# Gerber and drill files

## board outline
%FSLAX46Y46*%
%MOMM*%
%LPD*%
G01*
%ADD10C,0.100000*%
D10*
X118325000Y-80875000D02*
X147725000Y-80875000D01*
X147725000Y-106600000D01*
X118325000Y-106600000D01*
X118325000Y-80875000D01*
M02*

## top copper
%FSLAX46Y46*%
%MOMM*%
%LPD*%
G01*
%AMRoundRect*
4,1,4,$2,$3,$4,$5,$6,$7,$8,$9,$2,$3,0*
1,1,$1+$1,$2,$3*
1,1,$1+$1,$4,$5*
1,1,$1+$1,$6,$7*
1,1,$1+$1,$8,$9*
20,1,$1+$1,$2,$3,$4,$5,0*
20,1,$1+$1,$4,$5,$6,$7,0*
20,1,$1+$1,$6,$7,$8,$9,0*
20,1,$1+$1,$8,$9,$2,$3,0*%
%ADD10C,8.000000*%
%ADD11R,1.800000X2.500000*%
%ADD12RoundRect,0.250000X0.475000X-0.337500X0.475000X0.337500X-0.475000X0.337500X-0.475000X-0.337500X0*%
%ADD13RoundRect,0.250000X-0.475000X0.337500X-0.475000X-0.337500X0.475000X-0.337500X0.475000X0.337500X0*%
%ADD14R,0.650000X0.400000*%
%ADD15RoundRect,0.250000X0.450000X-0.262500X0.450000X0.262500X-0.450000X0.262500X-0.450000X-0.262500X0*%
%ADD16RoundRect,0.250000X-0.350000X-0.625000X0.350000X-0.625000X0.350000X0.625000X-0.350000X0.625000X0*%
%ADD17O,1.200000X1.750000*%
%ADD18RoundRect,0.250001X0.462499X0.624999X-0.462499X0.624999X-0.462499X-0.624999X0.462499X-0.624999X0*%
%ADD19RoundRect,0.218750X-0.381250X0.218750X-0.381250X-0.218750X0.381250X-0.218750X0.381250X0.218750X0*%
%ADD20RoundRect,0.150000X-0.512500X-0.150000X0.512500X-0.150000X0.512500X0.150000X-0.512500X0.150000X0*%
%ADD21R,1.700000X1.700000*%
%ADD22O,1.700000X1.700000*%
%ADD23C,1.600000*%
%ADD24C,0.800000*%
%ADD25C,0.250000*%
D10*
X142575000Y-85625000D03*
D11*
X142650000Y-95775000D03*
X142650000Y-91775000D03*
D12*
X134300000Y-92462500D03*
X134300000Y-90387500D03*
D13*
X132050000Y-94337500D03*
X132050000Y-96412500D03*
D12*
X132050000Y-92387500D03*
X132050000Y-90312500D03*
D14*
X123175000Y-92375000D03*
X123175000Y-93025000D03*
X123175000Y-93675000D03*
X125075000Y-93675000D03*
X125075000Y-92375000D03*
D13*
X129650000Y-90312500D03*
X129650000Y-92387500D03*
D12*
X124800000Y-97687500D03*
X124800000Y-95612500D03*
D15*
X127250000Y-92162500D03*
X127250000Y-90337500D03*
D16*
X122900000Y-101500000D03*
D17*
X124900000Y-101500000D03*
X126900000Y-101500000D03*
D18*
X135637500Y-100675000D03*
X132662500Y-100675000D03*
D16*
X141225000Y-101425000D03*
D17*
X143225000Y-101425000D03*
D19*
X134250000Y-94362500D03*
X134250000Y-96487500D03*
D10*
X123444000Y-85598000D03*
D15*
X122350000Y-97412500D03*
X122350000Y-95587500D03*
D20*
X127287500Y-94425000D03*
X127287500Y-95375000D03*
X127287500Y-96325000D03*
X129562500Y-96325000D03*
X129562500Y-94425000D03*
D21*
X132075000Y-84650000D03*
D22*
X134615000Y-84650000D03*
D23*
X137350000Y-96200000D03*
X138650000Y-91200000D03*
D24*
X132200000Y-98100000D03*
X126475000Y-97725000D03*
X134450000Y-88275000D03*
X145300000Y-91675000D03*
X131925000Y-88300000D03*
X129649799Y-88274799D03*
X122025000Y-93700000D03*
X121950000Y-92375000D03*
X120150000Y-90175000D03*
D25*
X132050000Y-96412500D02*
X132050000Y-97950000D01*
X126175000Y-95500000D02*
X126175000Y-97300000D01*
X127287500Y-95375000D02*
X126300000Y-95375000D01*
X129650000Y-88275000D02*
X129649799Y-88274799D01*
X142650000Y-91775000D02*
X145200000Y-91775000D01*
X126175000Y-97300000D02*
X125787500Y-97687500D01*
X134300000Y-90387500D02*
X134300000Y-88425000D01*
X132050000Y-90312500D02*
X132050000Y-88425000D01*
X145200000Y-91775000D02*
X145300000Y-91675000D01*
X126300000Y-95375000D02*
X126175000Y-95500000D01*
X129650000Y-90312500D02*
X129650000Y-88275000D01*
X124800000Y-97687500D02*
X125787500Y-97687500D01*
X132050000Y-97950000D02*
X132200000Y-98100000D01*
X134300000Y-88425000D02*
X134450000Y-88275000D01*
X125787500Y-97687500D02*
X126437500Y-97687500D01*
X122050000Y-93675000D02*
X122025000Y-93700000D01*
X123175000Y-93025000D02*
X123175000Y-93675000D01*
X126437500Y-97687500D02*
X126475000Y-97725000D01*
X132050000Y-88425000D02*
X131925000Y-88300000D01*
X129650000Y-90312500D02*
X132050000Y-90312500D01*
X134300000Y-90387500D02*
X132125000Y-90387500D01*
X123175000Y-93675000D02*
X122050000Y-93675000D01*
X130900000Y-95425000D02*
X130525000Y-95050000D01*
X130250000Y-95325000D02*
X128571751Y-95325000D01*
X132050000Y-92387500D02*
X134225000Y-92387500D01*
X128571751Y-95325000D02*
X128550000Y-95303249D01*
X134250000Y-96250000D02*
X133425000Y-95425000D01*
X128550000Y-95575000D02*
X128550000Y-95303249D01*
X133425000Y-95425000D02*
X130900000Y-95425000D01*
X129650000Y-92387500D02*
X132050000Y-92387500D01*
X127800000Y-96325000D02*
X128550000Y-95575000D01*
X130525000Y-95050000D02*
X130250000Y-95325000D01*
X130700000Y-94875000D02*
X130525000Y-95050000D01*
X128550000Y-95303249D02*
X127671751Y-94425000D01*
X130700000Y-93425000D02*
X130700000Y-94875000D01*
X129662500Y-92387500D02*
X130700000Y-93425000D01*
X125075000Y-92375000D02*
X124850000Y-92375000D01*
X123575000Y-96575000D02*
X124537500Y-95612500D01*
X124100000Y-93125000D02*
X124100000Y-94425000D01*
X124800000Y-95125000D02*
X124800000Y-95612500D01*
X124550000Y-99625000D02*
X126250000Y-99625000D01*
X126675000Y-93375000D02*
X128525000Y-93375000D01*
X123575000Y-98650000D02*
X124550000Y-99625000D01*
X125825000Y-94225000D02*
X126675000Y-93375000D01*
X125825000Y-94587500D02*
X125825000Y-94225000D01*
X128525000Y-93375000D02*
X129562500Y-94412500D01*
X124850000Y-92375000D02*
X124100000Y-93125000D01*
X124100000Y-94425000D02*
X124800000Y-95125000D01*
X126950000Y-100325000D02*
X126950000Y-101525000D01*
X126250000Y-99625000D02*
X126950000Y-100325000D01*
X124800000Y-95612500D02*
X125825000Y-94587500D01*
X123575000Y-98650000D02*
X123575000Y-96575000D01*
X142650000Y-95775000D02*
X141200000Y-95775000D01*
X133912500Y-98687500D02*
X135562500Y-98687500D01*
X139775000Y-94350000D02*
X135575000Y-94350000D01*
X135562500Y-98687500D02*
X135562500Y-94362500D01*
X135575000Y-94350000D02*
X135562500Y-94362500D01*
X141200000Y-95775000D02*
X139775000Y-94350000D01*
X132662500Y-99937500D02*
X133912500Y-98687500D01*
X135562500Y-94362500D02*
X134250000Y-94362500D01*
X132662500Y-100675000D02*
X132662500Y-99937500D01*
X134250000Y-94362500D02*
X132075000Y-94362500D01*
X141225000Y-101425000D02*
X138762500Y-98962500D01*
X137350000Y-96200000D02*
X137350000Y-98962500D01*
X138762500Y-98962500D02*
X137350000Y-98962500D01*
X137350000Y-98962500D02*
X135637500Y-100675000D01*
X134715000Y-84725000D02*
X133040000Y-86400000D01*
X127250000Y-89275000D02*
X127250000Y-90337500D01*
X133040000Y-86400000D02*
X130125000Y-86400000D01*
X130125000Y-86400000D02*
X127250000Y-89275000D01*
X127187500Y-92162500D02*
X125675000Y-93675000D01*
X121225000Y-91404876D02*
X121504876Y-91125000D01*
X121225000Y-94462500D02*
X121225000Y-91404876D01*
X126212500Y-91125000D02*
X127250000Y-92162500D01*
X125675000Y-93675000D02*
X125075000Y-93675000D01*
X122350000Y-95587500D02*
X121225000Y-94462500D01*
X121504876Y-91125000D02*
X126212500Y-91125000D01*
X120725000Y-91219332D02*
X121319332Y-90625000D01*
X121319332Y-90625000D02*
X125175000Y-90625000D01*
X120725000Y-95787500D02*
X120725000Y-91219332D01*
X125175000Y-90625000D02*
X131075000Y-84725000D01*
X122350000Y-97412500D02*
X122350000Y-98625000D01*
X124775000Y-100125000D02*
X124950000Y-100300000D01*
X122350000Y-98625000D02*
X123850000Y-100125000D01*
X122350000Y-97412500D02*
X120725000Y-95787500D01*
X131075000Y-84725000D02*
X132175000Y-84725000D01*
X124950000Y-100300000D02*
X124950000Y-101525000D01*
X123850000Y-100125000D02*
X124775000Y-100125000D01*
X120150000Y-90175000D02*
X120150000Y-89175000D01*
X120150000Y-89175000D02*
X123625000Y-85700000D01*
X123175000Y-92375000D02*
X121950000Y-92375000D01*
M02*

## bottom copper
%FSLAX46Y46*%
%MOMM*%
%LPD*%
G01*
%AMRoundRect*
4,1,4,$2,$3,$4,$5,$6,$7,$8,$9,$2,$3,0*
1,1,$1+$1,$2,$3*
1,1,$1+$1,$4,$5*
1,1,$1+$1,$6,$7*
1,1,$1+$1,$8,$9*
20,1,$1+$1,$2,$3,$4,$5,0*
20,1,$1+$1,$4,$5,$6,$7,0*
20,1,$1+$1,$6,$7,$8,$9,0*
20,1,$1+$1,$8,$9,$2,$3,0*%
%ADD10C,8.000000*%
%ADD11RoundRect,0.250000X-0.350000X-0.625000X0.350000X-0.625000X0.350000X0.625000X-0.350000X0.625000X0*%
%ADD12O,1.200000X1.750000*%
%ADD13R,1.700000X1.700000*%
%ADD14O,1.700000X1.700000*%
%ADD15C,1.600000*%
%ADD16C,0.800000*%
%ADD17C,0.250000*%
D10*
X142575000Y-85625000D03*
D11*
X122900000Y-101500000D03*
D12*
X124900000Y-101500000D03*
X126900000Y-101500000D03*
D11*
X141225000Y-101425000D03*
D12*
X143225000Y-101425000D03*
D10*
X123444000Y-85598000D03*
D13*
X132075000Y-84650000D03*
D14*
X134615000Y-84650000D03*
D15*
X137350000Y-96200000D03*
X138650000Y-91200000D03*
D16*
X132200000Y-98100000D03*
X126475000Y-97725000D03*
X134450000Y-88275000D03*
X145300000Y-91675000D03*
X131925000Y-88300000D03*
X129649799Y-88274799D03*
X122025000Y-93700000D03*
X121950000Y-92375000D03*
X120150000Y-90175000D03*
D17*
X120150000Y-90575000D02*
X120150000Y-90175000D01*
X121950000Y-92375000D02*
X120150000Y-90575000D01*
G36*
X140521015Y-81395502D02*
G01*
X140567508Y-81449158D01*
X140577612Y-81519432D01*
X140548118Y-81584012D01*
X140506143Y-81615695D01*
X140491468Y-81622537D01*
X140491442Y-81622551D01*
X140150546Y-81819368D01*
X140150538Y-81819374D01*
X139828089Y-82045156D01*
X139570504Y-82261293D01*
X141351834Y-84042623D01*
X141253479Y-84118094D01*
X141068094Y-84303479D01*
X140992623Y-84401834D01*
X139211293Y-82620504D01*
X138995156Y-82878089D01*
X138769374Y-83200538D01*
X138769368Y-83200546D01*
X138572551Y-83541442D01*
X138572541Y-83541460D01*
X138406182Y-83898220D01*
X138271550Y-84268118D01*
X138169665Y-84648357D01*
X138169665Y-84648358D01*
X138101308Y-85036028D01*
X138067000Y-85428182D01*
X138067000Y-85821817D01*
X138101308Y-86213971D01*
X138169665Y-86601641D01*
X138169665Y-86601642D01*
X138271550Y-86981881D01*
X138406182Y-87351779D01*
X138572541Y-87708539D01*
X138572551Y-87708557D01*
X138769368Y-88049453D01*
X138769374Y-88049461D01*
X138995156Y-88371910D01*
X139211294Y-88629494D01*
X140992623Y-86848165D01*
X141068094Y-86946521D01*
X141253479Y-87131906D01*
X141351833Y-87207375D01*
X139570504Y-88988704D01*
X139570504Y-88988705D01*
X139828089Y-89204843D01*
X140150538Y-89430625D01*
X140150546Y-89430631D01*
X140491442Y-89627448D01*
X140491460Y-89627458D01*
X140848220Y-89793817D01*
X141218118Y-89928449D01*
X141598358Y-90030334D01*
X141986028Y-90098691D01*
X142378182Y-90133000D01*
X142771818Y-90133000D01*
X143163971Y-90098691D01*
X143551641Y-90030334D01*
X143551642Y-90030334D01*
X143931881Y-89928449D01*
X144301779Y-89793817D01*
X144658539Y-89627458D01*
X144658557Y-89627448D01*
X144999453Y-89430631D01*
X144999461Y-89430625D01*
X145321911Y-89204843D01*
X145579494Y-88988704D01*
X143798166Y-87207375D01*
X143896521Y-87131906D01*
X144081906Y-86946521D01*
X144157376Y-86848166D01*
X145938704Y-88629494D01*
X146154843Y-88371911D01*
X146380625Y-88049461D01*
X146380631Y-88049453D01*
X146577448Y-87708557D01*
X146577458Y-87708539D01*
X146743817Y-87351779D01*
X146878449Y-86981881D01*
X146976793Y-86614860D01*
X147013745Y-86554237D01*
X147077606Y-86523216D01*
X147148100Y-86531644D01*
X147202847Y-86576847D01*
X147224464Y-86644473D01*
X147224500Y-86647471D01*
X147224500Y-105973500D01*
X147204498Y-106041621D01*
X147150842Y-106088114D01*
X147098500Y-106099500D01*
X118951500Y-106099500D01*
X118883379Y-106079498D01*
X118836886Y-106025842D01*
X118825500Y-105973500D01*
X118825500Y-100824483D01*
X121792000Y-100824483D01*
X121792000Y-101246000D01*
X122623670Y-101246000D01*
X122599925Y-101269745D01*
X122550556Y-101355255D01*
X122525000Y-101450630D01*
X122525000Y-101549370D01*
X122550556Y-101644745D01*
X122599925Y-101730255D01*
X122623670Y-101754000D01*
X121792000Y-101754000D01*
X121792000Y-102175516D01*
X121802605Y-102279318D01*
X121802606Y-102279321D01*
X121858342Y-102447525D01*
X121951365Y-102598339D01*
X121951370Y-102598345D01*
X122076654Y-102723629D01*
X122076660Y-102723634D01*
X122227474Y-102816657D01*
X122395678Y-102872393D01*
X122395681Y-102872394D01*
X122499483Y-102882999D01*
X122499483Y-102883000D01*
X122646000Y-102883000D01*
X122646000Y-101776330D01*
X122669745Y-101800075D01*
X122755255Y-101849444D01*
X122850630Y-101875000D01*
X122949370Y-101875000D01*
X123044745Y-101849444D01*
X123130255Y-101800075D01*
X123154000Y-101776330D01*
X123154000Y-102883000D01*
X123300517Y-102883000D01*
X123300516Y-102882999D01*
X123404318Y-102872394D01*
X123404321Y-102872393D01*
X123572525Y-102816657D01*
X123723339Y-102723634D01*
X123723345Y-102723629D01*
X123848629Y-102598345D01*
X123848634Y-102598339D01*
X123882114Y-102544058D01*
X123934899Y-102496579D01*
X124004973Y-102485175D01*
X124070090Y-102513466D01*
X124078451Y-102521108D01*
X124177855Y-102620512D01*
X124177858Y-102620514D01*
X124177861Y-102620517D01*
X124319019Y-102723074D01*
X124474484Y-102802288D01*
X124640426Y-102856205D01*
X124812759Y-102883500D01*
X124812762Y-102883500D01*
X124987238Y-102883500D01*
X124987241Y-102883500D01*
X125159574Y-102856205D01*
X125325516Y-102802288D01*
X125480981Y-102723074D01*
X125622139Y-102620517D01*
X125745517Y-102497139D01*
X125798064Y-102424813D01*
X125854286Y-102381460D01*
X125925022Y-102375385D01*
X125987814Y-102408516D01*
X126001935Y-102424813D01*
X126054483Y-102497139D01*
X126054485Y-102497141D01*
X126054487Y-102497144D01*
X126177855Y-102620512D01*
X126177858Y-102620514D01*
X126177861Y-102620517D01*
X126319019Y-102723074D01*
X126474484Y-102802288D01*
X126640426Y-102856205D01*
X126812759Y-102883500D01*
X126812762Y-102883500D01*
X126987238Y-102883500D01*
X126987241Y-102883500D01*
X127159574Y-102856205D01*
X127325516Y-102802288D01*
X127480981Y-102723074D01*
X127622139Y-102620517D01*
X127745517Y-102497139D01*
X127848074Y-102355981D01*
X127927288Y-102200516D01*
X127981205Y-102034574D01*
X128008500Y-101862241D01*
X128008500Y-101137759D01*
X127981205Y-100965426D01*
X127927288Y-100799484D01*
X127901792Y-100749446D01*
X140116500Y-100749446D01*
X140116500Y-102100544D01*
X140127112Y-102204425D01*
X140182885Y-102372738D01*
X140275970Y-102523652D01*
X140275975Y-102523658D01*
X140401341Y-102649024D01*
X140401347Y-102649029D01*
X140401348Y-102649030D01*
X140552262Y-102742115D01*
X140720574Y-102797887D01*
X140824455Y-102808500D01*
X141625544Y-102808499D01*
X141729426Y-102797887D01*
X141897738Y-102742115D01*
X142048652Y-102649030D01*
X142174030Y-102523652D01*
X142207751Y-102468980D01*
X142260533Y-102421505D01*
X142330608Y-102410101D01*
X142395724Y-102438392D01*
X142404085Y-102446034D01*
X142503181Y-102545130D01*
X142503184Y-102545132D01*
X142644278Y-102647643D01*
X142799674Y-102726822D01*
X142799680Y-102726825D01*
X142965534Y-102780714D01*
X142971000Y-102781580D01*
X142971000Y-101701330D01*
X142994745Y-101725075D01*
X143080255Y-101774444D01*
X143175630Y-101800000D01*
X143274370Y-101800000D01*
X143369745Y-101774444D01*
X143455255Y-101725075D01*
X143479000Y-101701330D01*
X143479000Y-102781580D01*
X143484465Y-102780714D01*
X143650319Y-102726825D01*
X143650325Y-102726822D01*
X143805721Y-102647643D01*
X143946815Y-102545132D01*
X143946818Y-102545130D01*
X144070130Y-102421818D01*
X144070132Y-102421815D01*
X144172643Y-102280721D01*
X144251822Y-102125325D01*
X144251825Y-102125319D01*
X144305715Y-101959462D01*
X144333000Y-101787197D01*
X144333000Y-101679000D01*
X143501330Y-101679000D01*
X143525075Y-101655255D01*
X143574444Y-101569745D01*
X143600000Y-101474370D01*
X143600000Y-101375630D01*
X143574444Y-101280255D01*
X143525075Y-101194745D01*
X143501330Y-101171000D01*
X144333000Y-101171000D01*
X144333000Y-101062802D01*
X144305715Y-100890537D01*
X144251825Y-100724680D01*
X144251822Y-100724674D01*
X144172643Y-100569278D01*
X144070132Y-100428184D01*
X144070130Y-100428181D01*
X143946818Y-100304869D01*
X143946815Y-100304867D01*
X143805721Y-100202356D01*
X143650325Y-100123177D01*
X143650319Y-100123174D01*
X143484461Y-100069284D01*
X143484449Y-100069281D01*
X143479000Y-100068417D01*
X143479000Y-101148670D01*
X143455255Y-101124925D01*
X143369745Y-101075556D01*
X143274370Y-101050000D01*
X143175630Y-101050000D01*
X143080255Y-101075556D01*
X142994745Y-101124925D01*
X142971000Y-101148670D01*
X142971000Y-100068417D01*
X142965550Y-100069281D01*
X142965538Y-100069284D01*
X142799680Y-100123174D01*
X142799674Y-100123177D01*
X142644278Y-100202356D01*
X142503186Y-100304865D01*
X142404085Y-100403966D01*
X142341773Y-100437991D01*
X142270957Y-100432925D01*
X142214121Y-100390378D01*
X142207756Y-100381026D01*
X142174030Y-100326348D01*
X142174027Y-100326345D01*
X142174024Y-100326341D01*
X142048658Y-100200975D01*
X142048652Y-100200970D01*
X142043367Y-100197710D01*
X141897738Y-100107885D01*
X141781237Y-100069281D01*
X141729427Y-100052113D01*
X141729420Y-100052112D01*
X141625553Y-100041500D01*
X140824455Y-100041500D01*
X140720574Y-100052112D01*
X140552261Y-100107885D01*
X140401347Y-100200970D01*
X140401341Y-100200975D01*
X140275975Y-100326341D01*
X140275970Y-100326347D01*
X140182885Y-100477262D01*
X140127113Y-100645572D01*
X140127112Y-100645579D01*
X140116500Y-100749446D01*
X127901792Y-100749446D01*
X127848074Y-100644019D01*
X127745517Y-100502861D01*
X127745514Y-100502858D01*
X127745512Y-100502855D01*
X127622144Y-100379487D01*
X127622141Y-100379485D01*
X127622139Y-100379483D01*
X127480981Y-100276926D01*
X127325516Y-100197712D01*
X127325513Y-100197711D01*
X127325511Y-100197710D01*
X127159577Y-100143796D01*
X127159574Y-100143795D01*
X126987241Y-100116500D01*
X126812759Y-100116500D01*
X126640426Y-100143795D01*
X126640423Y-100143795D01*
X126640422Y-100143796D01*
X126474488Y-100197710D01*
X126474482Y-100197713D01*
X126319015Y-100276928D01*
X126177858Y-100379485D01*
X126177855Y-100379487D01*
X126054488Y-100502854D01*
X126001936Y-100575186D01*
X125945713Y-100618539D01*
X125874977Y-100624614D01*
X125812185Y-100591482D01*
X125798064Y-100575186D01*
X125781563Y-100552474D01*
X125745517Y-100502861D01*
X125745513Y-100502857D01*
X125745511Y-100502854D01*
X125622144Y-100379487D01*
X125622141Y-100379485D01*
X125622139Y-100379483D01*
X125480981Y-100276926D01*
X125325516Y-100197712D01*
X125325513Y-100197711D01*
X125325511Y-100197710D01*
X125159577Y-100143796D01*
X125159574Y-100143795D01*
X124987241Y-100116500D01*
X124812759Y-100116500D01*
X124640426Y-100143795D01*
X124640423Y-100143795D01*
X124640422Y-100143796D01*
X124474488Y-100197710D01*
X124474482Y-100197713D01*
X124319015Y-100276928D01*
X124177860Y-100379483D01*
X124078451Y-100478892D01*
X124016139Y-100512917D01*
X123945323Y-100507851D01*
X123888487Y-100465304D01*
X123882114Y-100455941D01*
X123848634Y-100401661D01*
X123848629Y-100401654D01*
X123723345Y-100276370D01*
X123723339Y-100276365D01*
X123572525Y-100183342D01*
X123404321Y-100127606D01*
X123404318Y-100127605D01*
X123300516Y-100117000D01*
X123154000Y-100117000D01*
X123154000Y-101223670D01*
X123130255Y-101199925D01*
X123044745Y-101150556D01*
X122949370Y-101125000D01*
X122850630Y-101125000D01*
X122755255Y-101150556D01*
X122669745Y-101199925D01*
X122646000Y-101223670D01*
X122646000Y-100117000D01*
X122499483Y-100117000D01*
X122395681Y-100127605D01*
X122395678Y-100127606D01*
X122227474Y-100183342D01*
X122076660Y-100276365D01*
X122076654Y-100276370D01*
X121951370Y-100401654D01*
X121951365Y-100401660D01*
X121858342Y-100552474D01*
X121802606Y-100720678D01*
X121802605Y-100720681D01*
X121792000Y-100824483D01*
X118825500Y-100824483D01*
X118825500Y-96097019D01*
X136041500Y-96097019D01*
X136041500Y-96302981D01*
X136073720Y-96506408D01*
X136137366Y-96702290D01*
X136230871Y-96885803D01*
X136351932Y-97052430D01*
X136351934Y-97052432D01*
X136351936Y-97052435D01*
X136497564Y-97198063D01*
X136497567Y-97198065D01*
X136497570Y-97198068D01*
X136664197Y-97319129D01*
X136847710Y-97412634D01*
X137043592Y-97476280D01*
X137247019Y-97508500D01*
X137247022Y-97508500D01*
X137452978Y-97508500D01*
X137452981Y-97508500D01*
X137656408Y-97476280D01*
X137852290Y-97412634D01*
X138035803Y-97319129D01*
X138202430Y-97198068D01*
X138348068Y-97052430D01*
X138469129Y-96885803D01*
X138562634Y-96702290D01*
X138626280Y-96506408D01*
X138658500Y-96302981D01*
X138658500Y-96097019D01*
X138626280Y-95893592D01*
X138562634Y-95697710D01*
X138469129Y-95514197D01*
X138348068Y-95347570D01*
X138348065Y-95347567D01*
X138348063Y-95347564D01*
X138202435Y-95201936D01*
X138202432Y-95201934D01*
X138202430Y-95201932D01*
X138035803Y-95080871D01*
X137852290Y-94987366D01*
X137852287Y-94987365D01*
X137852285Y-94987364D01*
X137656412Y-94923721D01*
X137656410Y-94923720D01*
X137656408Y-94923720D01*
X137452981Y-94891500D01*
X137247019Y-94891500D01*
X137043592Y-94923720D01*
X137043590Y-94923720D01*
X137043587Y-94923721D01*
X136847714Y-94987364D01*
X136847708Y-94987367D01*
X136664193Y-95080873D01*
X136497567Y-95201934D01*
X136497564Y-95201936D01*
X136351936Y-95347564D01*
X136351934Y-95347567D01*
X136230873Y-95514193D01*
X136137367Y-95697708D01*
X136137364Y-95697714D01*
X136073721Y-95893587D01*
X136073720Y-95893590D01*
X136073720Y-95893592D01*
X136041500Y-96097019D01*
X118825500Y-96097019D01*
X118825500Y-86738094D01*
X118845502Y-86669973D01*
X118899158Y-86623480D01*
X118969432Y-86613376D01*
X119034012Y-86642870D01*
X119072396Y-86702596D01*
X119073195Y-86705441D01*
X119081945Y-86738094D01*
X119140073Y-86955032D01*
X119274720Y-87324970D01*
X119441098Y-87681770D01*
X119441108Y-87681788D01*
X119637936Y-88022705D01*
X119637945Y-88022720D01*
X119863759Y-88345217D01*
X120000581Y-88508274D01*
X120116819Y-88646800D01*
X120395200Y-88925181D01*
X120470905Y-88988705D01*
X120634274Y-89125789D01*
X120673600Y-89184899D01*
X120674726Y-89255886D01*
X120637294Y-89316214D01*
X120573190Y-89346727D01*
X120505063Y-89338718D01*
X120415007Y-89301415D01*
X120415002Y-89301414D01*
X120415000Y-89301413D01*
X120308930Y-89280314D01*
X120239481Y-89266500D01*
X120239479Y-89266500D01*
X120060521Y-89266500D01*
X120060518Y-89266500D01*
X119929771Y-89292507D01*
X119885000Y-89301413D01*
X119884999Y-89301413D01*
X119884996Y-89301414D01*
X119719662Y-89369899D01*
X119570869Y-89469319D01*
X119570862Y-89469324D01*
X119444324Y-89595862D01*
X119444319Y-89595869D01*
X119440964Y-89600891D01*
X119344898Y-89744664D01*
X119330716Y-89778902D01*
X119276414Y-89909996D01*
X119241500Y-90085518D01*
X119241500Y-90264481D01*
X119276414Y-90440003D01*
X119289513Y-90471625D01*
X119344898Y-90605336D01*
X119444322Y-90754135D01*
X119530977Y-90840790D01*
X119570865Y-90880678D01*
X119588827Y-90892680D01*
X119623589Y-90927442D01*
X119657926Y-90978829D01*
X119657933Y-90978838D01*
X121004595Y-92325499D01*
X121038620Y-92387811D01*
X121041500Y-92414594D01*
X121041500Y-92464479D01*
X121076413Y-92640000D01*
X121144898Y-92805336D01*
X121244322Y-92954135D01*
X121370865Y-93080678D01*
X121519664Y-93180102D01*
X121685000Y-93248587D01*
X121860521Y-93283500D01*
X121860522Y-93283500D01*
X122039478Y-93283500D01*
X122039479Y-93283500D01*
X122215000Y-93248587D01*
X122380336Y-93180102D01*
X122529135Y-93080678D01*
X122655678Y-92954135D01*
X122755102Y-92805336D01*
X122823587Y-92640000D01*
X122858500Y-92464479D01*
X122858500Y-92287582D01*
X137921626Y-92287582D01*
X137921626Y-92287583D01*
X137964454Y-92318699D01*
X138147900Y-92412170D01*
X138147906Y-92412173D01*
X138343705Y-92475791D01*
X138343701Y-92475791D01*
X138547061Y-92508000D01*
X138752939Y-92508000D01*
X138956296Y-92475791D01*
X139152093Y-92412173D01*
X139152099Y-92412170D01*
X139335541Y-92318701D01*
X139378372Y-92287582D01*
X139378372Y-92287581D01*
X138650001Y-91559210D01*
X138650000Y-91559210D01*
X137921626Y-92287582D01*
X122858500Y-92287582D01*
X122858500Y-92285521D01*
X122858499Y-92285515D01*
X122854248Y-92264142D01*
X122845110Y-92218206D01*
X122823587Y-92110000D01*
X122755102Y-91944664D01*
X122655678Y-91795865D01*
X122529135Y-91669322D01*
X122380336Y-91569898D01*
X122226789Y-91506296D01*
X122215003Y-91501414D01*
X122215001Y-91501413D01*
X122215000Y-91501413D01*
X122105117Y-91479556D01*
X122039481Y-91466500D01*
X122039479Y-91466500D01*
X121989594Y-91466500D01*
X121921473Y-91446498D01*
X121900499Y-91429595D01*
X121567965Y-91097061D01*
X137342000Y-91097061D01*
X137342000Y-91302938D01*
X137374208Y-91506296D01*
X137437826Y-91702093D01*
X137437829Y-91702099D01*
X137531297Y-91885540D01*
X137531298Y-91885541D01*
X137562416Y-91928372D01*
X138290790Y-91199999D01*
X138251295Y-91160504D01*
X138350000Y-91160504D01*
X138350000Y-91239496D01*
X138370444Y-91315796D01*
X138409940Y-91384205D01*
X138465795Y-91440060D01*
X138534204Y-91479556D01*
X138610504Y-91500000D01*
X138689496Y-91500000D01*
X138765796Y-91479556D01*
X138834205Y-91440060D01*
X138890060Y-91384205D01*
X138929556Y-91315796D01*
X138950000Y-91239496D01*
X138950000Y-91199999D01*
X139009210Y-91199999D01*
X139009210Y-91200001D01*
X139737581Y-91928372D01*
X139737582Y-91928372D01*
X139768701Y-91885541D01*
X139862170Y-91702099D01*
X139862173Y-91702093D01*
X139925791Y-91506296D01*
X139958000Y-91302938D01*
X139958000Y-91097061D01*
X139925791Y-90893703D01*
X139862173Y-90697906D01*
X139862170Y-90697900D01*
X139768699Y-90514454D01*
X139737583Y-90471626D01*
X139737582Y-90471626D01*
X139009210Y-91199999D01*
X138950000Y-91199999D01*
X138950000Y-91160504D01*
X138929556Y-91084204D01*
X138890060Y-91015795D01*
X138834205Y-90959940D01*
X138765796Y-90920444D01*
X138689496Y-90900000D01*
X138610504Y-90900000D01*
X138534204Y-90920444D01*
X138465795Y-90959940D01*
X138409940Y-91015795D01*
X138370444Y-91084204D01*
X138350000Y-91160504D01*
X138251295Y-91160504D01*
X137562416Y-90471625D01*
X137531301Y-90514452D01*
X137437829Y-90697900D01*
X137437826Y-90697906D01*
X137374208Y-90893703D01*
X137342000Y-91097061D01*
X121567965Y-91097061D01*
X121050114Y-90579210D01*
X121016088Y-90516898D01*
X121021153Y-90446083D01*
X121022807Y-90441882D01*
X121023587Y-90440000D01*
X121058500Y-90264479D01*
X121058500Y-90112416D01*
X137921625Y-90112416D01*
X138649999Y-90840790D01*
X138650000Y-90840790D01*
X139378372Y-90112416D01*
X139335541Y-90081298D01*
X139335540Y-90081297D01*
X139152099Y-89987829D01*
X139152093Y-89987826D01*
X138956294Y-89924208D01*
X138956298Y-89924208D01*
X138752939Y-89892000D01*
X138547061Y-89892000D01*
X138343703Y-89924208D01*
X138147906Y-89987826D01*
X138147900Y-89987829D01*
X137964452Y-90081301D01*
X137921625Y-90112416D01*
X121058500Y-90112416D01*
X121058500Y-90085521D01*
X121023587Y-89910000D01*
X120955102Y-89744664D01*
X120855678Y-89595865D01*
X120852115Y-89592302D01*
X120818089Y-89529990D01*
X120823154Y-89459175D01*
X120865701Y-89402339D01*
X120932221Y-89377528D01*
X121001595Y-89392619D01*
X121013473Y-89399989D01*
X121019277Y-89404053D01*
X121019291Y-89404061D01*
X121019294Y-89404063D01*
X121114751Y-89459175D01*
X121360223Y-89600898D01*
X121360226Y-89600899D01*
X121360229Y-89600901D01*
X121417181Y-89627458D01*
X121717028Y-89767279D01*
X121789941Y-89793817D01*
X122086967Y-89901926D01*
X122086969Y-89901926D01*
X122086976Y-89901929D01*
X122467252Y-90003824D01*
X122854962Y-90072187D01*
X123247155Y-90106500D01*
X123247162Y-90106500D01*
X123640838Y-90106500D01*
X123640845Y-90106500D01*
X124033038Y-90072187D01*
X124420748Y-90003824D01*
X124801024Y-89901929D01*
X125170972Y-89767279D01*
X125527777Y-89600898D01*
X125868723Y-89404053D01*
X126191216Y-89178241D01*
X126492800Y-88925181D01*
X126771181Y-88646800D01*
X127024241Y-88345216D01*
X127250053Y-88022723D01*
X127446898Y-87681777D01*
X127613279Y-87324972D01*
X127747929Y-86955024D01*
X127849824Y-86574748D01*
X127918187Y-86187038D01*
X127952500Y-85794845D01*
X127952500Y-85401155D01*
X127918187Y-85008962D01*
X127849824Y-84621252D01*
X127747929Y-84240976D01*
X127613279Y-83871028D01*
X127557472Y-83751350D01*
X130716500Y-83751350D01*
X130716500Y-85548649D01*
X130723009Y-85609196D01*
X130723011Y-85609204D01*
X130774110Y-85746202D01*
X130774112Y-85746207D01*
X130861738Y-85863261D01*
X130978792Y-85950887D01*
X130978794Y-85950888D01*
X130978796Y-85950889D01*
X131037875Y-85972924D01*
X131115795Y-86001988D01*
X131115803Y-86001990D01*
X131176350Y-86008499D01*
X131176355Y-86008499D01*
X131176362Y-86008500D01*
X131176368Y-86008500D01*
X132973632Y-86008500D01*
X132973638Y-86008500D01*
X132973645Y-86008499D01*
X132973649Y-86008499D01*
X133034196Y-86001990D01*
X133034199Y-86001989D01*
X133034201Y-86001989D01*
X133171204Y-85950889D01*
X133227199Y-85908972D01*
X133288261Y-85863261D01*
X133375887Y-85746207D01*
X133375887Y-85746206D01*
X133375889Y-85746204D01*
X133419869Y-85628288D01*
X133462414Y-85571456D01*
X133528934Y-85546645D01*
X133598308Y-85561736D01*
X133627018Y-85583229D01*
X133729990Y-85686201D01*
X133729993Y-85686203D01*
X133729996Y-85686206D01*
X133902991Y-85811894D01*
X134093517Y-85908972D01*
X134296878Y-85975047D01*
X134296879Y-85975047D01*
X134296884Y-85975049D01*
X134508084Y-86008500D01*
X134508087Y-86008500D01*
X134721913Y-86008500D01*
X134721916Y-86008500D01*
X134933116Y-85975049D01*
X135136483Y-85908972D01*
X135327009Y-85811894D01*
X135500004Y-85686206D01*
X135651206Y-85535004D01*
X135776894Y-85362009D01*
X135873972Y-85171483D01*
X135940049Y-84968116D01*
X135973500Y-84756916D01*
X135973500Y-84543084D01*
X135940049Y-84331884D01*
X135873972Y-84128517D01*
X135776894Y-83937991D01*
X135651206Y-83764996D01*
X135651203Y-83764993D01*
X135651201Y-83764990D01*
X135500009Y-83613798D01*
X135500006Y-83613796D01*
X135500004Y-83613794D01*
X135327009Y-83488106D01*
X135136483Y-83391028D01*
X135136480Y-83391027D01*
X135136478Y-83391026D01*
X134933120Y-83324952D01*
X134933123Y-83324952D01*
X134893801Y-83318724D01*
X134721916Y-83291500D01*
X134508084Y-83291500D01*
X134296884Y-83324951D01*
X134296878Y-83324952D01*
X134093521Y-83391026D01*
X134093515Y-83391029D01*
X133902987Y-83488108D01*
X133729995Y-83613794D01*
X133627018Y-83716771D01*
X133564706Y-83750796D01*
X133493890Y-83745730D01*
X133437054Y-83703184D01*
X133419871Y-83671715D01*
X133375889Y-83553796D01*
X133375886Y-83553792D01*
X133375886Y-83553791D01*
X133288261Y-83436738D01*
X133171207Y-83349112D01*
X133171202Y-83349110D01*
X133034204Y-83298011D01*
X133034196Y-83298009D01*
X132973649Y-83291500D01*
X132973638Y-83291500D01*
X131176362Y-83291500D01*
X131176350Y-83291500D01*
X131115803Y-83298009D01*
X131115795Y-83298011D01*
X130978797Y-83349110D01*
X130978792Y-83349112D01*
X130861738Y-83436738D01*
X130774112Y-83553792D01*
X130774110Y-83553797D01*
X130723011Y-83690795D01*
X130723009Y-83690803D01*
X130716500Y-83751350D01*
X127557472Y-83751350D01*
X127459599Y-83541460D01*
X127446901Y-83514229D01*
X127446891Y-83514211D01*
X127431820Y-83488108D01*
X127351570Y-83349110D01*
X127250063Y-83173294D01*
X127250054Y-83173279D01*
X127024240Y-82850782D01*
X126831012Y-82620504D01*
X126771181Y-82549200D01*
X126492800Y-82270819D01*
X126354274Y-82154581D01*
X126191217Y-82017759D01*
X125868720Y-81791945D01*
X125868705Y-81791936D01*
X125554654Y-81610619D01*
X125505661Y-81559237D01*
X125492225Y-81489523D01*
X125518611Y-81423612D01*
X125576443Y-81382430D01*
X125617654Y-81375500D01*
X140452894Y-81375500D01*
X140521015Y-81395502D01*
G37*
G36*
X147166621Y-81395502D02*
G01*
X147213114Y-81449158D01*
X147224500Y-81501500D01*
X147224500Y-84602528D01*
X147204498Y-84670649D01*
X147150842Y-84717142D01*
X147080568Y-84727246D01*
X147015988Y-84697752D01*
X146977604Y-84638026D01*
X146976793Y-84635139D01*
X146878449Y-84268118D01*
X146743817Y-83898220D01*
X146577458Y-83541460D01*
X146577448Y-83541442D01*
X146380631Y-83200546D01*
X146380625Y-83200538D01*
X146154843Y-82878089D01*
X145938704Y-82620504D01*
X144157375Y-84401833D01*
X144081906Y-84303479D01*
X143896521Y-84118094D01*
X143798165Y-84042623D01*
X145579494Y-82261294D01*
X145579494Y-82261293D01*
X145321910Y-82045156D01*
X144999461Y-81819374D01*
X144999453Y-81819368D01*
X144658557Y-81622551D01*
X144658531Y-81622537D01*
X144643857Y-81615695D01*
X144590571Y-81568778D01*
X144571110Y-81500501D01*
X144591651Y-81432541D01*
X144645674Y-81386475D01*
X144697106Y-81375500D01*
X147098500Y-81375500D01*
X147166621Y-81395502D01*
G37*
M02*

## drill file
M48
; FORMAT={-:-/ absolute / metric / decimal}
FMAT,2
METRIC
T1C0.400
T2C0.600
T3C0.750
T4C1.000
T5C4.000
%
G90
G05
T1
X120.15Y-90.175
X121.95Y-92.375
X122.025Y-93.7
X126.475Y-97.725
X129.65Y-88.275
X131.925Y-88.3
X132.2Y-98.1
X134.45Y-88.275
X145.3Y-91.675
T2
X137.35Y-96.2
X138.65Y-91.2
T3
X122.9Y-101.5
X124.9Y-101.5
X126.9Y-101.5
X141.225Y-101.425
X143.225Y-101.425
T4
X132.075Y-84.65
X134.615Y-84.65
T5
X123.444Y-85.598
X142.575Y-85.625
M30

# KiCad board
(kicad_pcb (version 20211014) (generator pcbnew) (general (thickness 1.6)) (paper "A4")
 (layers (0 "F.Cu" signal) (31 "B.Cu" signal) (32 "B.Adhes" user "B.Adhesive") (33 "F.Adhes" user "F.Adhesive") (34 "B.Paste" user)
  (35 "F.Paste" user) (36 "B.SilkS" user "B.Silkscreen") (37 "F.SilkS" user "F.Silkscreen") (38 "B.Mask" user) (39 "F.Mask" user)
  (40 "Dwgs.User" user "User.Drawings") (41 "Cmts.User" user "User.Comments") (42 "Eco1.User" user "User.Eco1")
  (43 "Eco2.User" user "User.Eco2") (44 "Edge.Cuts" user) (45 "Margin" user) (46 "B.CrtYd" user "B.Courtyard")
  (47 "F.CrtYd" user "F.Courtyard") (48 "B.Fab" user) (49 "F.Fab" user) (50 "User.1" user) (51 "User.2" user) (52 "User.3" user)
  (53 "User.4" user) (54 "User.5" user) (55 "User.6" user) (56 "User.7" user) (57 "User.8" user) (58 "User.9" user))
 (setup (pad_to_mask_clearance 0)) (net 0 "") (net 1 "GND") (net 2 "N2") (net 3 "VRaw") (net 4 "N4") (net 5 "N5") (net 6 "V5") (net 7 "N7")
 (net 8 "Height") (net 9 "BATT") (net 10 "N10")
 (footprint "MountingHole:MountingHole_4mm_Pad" (layer "F.Cu") (at 142.575 85.625)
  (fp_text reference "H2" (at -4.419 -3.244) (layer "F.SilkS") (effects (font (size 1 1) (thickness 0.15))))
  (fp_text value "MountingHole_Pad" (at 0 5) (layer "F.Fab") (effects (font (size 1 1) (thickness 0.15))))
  (pad "1" thru_hole circle (at 0 0) (size 8 8) (drill 4) (layers *.Cu *.Mask) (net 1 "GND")))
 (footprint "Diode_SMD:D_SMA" (layer "F.Cu") (at 142.65 93.775 90)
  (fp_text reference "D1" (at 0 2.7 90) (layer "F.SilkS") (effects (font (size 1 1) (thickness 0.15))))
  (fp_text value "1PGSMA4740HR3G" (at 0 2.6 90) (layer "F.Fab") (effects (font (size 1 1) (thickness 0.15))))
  (pad "1" smd rect (at -2 0 90) (size 2.5 1.8) (layers "F.Cu" "F.Paste" "F.Mask") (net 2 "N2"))
  (pad "2" smd rect (at 2 0 90) (size 2.5 1.8) (layers "F.Cu" "F.Paste" "F.Mask") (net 1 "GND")))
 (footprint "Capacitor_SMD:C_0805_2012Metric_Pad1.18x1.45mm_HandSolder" (layer "F.Cu") (at 134.3 91.425 90)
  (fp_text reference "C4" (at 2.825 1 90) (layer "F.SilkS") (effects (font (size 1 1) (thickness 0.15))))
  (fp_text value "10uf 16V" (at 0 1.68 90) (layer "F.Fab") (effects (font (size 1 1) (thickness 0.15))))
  (pad "1" smd roundrect (at -1.0375 0 90) (size 1.175 1.45) (layers "F.Cu" "F.Paste" "F.Mask") (roundrect_rratio 0.2127659574)
   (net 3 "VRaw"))
  (pad "2" smd roundrect (at 1.0375 0 90) (size 1.175 1.45) (layers "F.Cu" "F.Paste" "F.Mask") (roundrect_rratio 0.2127659574) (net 1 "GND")))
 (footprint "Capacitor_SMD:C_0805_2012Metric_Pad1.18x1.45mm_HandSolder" (layer "F.Cu") (at 132.05 95.375 -90)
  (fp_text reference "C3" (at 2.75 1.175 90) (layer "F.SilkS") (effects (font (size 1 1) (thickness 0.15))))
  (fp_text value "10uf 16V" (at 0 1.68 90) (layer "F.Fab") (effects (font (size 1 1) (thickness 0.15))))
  (pad "1" smd roundrect (at -1.0375 0 270) (size 1.175 1.45) (layers "F.Cu" "F.Paste" "F.Mask") (roundrect_rratio 0.2127659574)
   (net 2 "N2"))
  (pad "2" smd roundrect (at 1.0375 0 270) (size 1.175 1.45) (layers "F.Cu" "F.Paste" "F.Mask") (roundrect_rratio 0.2127659574)
   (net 1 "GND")))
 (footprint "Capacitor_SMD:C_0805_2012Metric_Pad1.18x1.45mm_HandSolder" (layer "F.Cu") (at 132.05 91.35 90)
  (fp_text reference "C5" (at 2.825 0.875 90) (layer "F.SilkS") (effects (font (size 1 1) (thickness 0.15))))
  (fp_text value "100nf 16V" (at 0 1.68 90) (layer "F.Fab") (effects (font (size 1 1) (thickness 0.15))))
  (pad "1" smd roundrect (at -1.0375 0 90) (size 1.175 1.45) (layers "F.Cu" "F.Paste" "F.Mask") (roundrect_rratio 0.2127659574)
   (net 3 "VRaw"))
  (pad "2" smd roundrect (at 1.0375 0 90) (size 1.175 1.45) (layers "F.Cu" "F.Paste" "F.Mask") (roundrect_rratio 0.2127659574) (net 1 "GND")))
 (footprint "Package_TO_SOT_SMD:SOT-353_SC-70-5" (layer "F.Cu") (at 124.125 93.025)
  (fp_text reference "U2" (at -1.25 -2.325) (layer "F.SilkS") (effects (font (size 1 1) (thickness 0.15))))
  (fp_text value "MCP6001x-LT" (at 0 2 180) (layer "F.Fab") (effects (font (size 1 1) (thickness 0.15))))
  (pad "1" smd rect (at -0.95 -0.65) (size 0.65 0.4) (layers "F.Cu" "F.Paste" "F.Mask") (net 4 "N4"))
  (pad "2" smd rect (at -0.95 0) (size 0.65 0.4) (layers "F.Cu" "F.Paste" "F.Mask") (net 1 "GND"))
  (pad "3" smd rect (at -0.95 0.65) (size 0.65 0.4) (layers "F.Cu" "F.Paste" "F.Mask") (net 1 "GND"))
  (pad "4" smd rect (at 0.95 0.65) (size 0.65 0.4) (layers "F.Cu" "F.Paste" "F.Mask") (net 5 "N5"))
  (pad "5" smd rect (at 0.95 -0.65) (size 0.65 0.4) (layers "F.Cu" "F.Paste" "F.Mask") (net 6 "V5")))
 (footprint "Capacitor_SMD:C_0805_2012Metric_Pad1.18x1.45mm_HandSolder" (layer "F.Cu") (at 129.65 91.35 -90)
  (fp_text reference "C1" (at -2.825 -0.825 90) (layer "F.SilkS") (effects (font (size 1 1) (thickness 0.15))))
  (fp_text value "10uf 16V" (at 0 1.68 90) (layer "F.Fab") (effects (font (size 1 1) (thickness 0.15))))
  (pad "1" smd roundrect (at -1.0375 0 270) (size 1.175 1.45) (layers "F.Cu" "F.Paste" "F.Mask") (roundrect_rratio 0.2127659574)
   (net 1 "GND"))
  (pad "2" smd roundrect (at 1.0375 0 270) (size 1.175 1.45) (layers "F.Cu" "F.Paste" "F.Mask") (roundrect_rratio 0.2127659574)
   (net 3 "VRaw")))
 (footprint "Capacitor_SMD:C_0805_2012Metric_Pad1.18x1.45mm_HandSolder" (layer "F.Cu") (at 124.8 96.65 90)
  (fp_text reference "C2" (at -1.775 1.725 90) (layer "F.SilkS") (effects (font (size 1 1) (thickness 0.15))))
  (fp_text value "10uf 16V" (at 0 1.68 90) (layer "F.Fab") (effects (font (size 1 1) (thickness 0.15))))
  (pad "1" smd roundrect (at -1.0375 0 90) (size 1.175 1.45) (layers "F.Cu" "F.Paste" "F.Mask") (roundrect_rratio 0.2127659574)
   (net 1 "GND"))
  (pad "2" smd roundrect (at 1.0375 0 90) (size 1.175 1.45) (layers "F.Cu" "F.Paste" "F.Mask") (roundrect_rratio 0.2127659574) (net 6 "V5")))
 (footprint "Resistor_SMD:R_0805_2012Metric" (layer "F.Cu") (at 127.25 91.25 90)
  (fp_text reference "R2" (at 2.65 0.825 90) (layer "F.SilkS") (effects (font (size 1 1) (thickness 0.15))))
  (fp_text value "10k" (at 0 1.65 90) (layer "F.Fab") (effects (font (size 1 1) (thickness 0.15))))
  (pad "1" smd roundrect (at -0.9125 0 90) (size 1.025 1.4) (layers "F.Cu" "F.Paste" "F.Mask") (roundrect_rratio 0.243902439) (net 5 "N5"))
  (pad "2" smd roundrect (at 0.9125 0 90) (size 1.025 1.4) (layers "F.Cu" "F.Paste" "F.Mask") (roundrect_rratio 0.243902439) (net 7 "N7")))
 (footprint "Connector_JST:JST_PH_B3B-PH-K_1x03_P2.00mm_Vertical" (layer "F.Cu") (at 122.9 101.5)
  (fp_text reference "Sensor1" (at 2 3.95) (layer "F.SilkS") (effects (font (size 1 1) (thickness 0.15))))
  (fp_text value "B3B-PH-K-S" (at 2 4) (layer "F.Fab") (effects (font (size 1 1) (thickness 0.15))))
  (pad "1" thru_hole roundrect (at 0 0) (size 1.2 1.75) (drill 0.75) (layers *.Cu *.Mask) (roundrect_rratio 0.208333) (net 1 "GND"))
  (pad "2" thru_hole oval (at 2 0) (size 1.2 1.75) (drill 0.75) (layers *.Cu *.Mask) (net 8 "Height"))
  (pad "3" thru_hole oval (at 4 0) (size 1.2 1.75) (drill 0.75) (layers *.Cu *.Mask) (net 6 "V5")))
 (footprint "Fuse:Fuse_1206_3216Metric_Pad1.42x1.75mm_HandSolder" (layer "F.Cu") (at 134.15 100.675 180)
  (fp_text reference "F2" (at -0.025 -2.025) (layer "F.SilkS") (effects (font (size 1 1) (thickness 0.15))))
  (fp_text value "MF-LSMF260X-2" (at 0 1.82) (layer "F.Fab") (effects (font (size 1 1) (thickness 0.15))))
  (pad "1" smd roundrect (at -1.4875 0 180) (size 1.425 1.75) (layers "F.Cu" "F.Paste" "F.Mask") (roundrect_rratio 0.175439) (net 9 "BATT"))
  (pad "2" smd roundrect (at 1.4875 0 180) (size 1.425 1.75) (layers "F.Cu" "F.Paste" "F.Mask") (roundrect_rratio 0.175439) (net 2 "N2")))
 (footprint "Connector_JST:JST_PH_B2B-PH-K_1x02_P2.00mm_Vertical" (layer "F.Cu") (at 141.225 101.425)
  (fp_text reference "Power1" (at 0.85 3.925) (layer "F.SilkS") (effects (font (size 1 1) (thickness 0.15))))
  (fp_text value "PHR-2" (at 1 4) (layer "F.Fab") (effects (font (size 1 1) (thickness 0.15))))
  (pad "1" thru_hole roundrect (at 0 0) (size 1.2 1.75) (drill 0.75) (layers *.Cu *.Mask) (roundrect_rratio 0.208333) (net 9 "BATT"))
  (pad "2" thru_hole oval (at 2 0) (size 1.2 1.75) (drill 0.75) (layers *.Cu *.Mask) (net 1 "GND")))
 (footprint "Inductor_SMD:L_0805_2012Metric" (layer "F.Cu") (at 134.25 95.425 -90)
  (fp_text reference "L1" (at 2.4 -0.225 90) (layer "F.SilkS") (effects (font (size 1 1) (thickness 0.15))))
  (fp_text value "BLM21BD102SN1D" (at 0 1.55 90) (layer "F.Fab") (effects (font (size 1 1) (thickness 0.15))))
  (pad "1" smd roundrect (at -1.0625 0 270) (size 0.875 1.2) (layers "F.Cu" "F.Paste" "F.Mask") (roundrect_rratio 0.25) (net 2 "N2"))
  (pad "2" smd roundrect (at 1.0625 0 270) (size 0.875 1.2) (layers "F.Cu" "F.Paste" "F.Mask") (roundrect_rratio 0.25) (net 3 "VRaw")))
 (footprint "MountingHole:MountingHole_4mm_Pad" (layer "F.Cu") (at 123.444 85.598)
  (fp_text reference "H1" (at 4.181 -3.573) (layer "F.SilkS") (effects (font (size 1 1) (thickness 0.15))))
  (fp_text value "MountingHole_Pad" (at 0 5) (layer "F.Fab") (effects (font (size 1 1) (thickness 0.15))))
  (pad "1" thru_hole circle (at 0 0) (size 8 8) (drill 4) (layers *.Cu *.Mask) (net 4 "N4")))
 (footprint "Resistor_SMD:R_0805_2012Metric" (layer "F.Cu") (at 122.35 96.5 90)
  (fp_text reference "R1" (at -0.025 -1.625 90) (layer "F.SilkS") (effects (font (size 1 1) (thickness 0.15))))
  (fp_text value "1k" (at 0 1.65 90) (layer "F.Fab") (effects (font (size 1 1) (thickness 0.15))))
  (pad "1" smd roundrect (at -0.9125 0 90) (size 1.025 1.4) (layers "F.Cu" "F.Paste" "F.Mask") (roundrect_rratio 0.243902439)
   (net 8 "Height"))
  (pad "2" smd roundrect (at 0.9125 0 90) (size 1.025 1.4) (layers "F.Cu" "F.Paste" "F.Mask") (roundrect_rratio 0.243902439) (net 5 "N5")))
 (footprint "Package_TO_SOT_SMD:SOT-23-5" (layer "F.Cu") (at 128.425 95.375)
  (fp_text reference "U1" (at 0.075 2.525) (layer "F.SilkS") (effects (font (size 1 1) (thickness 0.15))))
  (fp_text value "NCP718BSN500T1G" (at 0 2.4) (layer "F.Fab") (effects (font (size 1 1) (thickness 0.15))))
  (pad "1" smd roundrect (at -1.1375 -0.95) (size 1.325 0.6) (layers "F.Cu" "F.Paste" "F.Mask") (roundrect_rratio 0.25) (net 3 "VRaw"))
  (pad "2" smd roundrect (at -1.1375 0) (size 1.325 0.6) (layers "F.Cu" "F.Paste" "F.Mask") (roundrect_rratio 0.25) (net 1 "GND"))
  (pad "3" smd roundrect (at -1.1375 0.95) (size 1.325 0.6) (layers "F.Cu" "F.Paste" "F.Mask") (roundrect_rratio 0.25) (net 3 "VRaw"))
  (pad "4" smd roundrect (at 1.1375 0.95) (size 1.325 0.6) (layers "F.Cu" "F.Paste" "F.Mask") (roundrect_rratio 0.25) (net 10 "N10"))
  (pad "5" smd roundrect (at 1.1375 -0.95) (size 1.325 0.6) (layers "F.Cu" "F.Paste" "F.Mask") (roundrect_rratio 0.25) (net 6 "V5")))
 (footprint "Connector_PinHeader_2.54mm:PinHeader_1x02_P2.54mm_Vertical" (layer "F.Cu") (at 132.075 84.65 90)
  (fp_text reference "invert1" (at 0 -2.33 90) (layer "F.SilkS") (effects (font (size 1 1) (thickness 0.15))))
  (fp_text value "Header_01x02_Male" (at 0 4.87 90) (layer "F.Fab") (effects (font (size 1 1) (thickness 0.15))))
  (pad "1" thru_hole rect (at 0 0 90) (size 1.7 1.7) (drill 1) (layers *.Cu *.Mask) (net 8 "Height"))
  (pad "2" thru_hole oval (at 0 2.54 90) (size 1.7 1.7) (drill 1) (layers *.Cu *.Mask) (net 7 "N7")))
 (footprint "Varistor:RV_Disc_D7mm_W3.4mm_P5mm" (layer "F.Cu") (at 137.35 96.2 90)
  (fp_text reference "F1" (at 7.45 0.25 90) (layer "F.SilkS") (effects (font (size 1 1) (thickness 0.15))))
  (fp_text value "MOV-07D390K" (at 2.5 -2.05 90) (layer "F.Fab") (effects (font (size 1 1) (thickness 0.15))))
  (pad "1" thru_hole circle (at 0 0 90) (size 1.6 1.6) (drill 0.6) (layers *.Cu *.Mask) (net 9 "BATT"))
  (pad "2" thru_hole circle (at 5 1.3 90) (size 1.6 1.6) (drill 0.6) (layers *.Cu *.Mask) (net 1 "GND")))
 (gr_rect (start 118.325 80.875) (end 147.725 106.6) (layer "Edge.Cuts") (width 0.1) (fill none))
 (segment (start 132.05 96.4125) (end 132.05 97.95) (width 0.25) (layer "F.Cu") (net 1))
 (segment (start 126.175 95.5) (end 126.175 97.3) (width 0.25) (layer "F.Cu") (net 1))
 (segment (start 127.2875 95.375) (end 126.3 95.375) (width 0.25) (layer "F.Cu") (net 1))
 (segment (start 129.65 88.275) (end 129.649799 88.274799) (width 0.25) (layer "F.Cu") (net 1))
 (segment (start 142.65 91.775) (end 145.2 91.775) (width 0.25) (layer "F.Cu") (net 1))
 (segment (start 126.175 97.3) (end 125.7875 97.6875) (width 0.25) (layer "F.Cu") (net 1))
 (segment (start 134.3 90.3875) (end 134.3 88.425) (width 0.25) (layer "F.Cu") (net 1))
 (segment (start 132.05 90.3125) (end 132.05 88.425) (width 0.25) (layer "F.Cu") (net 1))
 (segment (start 145.2 91.775) (end 145.3 91.675) (width 0.25) (layer "F.Cu") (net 1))
 (segment (start 126.3 95.375) (end 126.175 95.5) (width 0.25) (layer "F.Cu") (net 1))
 (segment (start 129.65 90.3125) (end 129.65 88.275) (width 0.25) (layer "F.Cu") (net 1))
 (segment (start 124.8 97.6875) (end 125.7875 97.6875) (width 0.25) (layer "F.Cu") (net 1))
 (segment (start 132.05 97.95) (end 132.2 98.1) (width 0.25) (layer "F.Cu") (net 1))
 (segment (start 134.3 88.425) (end 134.45 88.275) (width 0.25) (layer "F.Cu") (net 1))
 (segment (start 125.7875 97.6875) (end 126.4375 97.6875) (width 0.25) (layer "F.Cu") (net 1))
 (segment (start 122.05 93.675) (end 122.025 93.7) (width 0.25) (layer "F.Cu") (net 1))
 (segment (start 123.175 93.025) (end 123.175 93.675) (width 0.25) (layer "F.Cu") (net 1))
 (segment (start 126.4375 97.6875) (end 126.475 97.725) (width 0.25) (layer "F.Cu") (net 1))
 (segment (start 132.05 88.425) (end 131.925 88.3) (width 0.25) (layer "F.Cu") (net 1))
 (segment (start 129.65 90.3125) (end 132.05 90.3125) (width 0.25) (layer "F.Cu") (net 1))
 (segment (start 134.3 90.3875) (end 132.125 90.3875) (width 0.25) (layer "F.Cu") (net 1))
 (segment (start 123.175 93.675) (end 122.05 93.675) (width 0.25) (layer "F.Cu") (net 1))
 (via (at 132.2 98.1) (size 0.8) (drill 0.4) (layers "F.Cu" "B.Cu") (free) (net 1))
 (via (at 126.475 97.725) (size 0.8) (drill 0.4) (layers "F.Cu" "B.Cu") (free) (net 1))
 (via (at 134.45 88.275) (size 0.8) (drill 0.4) (layers "F.Cu" "B.Cu") (free) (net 1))
 (via (at 145.3 91.675) (size 0.8) (drill 0.4) (layers "F.Cu" "B.Cu") (free) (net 1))
 (via (at 131.925 88.3) (size 0.8) (drill 0.4) (layers "F.Cu" "B.Cu") (free) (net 1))
 (via (at 129.649799 88.274799) (size 0.8) (drill 0.4) (layers "F.Cu" "B.Cu") (free) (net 1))
 (via (at 122.025 93.7) (size 0.8) (drill 0.4) (layers "F.Cu" "B.Cu") (free) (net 1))
 (segment (start 130.9 95.425) (end 130.525 95.05) (width 0.25) (layer "F.Cu") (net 3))
 (segment (start 130.25 95.325) (end 128.571751 95.325) (width 0.25) (layer "F.Cu") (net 3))
 (segment (start 132.05 92.3875) (end 134.225 92.3875) (width 0.25) (layer "F.Cu") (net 3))
 (segment (start 128.571751 95.325) (end 128.55 95.303249) (width 0.25) (layer "F.Cu") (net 3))
 (segment (start 134.25 96.25) (end 133.425 95.425) (width 0.25) (layer "F.Cu") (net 3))
 (segment (start 128.55 95.575) (end 128.55 95.303249) (width 0.25) (layer "F.Cu") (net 3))
 (segment (start 133.425 95.425) (end 130.9 95.425) (width 0.25) (layer "F.Cu") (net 3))
 (segment (start 129.65 92.3875) (end 132.05 92.3875) (width 0.25) (layer "F.Cu") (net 3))
 (segment (start 127.8 96.325) (end 128.55 95.575) (width 0.25) (layer "F.Cu") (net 3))
 (segment (start 130.525 95.05) (end 130.25 95.325) (width 0.25) (layer "F.Cu") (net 3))
 (segment (start 130.7 94.875) (end 130.525 95.05) (width 0.25) (layer "F.Cu") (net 3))
 (segment (start 128.55 95.303249) (end 127.671751 94.425) (width 0.25) (layer "F.Cu") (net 3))
 (segment (start 130.7 93.425) (end 130.7 94.875) (width 0.25) (layer "F.Cu") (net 3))
 (segment (start 129.6625 92.3875) (end 130.7 93.425) (width 0.25) (layer "F.Cu") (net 3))
 (segment (start 125.075 92.375) (end 124.85 92.375) (width 0.25) (layer "F.Cu") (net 6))
 (segment (start 123.575 96.575) (end 124.5375 95.6125) (width 0.25) (layer "F.Cu") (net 6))
 (segment (start 124.1 93.125) (end 124.1 94.425) (width 0.25) (layer "F.Cu") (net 6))
 (segment (start 124.8 95.125) (end 124.8 95.6125) (width 0.25) (layer "F.Cu") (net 6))
 (segment (start 124.55 99.625) (end 126.25 99.625) (width 0.25) (layer "F.Cu") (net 6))
 (segment (start 126.675 93.375) (end 128.525 93.375) (width 0.25) (layer "F.Cu") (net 6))
 (segment (start 123.575 98.65) (end 124.55 99.625) (width 0.25) (layer "F.Cu") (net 6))
 (segment (start 125.825 94.225) (end 126.675 93.375) (width 0.25) (layer "F.Cu") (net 6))
 (segment (start 125.825 94.5875) (end 125.825 94.225) (width 0.25) (layer "F.Cu") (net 6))
 (segment (start 128.525 93.375) (end 129.5625 94.4125) (width 0.25) (layer "F.Cu") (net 6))
 (segment (start 124.85 92.375) (end 124.1 93.125) (width 0.25) (layer "F.Cu") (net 6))
 (segment (start 124.1 94.425) (end 124.8 95.125) (width 0.25) (layer "F.Cu") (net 6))
 (segment (start 126.95 100.325) (end 126.95 101.525) (width 0.25) (layer "F.Cu") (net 6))
 (segment (start 126.25 99.625) (end 126.95 100.325) (width 0.25) (layer "F.Cu") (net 6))
 (segment (start 124.8 95.6125) (end 125.825 94.5875) (width 0.25) (layer "F.Cu") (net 6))
 (segment (start 123.575 98.65) (end 123.575 96.575) (width 0.25) (layer "F.Cu") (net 6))
 (segment (start 142.65 95.775) (end 141.2 95.775) (width 0.25) (layer "F.Cu") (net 2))
 (segment (start 133.9125 98.6875) (end 135.5625 98.6875) (width 0.25) (layer "F.Cu") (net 2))
 (segment (start 139.775 94.35) (end 135.575 94.35) (width 0.25) (layer "F.Cu") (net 2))
 (segment (start 135.5625 98.6875) (end 135.5625 94.3625) (width 0.25) (layer "F.Cu") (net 2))
 (segment (start 135.575 94.35) (end 135.5625 94.3625) (width 0.25) (layer "F.Cu") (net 2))
 (segment (start 141.2 95.775) (end 139.775 94.35) (width 0.25) (layer "F.Cu") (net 2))
 (segment (start 132.6625 99.9375) (end 133.9125 98.6875) (width 0.25) (layer "F.Cu") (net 2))
 (segment (start 135.5625 94.3625) (end 134.25 94.3625) (width 0.25) (layer "F.Cu") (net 2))
 (segment (start 132.6625 100.675) (end 132.6625 99.9375) (width 0.25) (layer "F.Cu") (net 2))
 (segment (start 134.25 94.3625) (end 132.075 94.3625) (width 0.25) (layer "F.Cu") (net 2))
 (segment (start 141.225 101.425) (end 138.7625 98.9625) (width 0.25) (layer "F.Cu") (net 9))
 (segment (start 137.35 96.2) (end 137.35 98.9625) (width 0.25) (layer "F.Cu") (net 9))
 (segment (start 138.7625 98.9625) (end 137.35 98.9625) (width 0.25) (layer "F.Cu") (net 9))
 (segment (start 137.35 98.9625) (end 135.6375 100.675) (width 0.25) (layer "F.Cu") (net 9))
 (segment (start 134.715 84.725) (end 133.04 86.4) (width 0.25) (layer "F.Cu") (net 7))
 (segment (start 127.25 89.275) (end 127.25 90.3375) (width 0.25) (layer "F.Cu") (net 7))
 (segment (start 133.04 86.4) (end 130.125 86.4) (width 0.25) (layer "F.Cu") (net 7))
 (segment (start 130.125 86.4) (end 127.25 89.275) (width 0.25) (layer "F.Cu") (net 7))
 (segment (start 127.1875 92.1625) (end 125.675 93.675) (width 0.25) (layer "F.Cu") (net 5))
 (segment (start 121.225 91.404876) (end 121.504876 91.125) (width 0.25) (layer "F.Cu") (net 5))
 (segment (start 121.225 94.4625) (end 121.225 91.404876) (width 0.25) (layer "F.Cu") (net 5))
 (segment (start 126.2125 91.125) (end 127.25 92.1625) (width 0.25) (layer "F.Cu") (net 5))
 (segment (start 125.675 93.675) (end 125.075 93.675) (width 0.25) (layer "F.Cu") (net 5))
 (segment (start 122.35 95.5875) (end 121.225 94.4625) (width 0.25) (layer "F.Cu") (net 5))
 (segment (start 121.504876 91.125) (end 126.2125 91.125) (width 0.25) (layer "F.Cu") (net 5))
 (segment (start 120.725 91.219332) (end 121.319332 90.625) (width 0.25) (layer "F.Cu") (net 8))
 (segment (start 121.319332 90.625) (end 125.175 90.625) (width 0.25) (layer "F.Cu") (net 8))
 (segment (start 120.725 95.7875) (end 120.725 91.219332) (width 0.25) (layer "F.Cu") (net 8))
 (segment (start 125.175 90.625) (end 131.075 84.725) (width 0.25) (layer "F.Cu") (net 8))
 (segment (start 122.35 97.4125) (end 122.35 98.625) (width 0.25) (layer "F.Cu") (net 8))
 (segment (start 124.775 100.125) (end 124.95 100.3) (width 0.25) (layer "F.Cu") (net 8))
 (segment (start 122.35 98.625) (end 123.85 100.125) (width 0.25) (layer "F.Cu") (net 8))
 (segment (start 122.35 97.4125) (end 120.725 95.7875) (width 0.25) (layer "F.Cu") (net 8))
 (segment (start 131.075 84.725) (end 132.175 84.725) (width 0.25) (layer "F.Cu") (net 8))
 (segment (start 124.95 100.3) (end 124.95 101.525) (width 0.25) (layer "F.Cu") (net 8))
 (segment (start 123.85 100.125) (end 124.775 100.125) (width 0.25) (layer "F.Cu") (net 8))
 (segment (start 120.15 90.175) (end 120.15 89.175) (width 0.25) (layer "F.Cu") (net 4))
 (segment (start 120.15 89.175) (end 123.625 85.7) (width 0.25) (layer "F.Cu") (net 4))
 (segment (start 123.175 92.375) (end 121.95 92.375) (width 0.25) (layer "F.Cu") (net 4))
 (via (at 121.95 92.375) (size 0.8) (drill 0.4) (layers "F.Cu" "B.Cu") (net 4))
 (via (at 120.15 90.175) (size 0.8) (drill 0.4) (layers "F.Cu" "B.Cu") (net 4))
 (segment (start 120.15 90.575) (end 120.15 90.175) (width 0.25) (layer "B.Cu") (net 4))
 (segment (start 121.95 92.375) (end 120.15 90.575) (width 0.25) (layer "B.Cu") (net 4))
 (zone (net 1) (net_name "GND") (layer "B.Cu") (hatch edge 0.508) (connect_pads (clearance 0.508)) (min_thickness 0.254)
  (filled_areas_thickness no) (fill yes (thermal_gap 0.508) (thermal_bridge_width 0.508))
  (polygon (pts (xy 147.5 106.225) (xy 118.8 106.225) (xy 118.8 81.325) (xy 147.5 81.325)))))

